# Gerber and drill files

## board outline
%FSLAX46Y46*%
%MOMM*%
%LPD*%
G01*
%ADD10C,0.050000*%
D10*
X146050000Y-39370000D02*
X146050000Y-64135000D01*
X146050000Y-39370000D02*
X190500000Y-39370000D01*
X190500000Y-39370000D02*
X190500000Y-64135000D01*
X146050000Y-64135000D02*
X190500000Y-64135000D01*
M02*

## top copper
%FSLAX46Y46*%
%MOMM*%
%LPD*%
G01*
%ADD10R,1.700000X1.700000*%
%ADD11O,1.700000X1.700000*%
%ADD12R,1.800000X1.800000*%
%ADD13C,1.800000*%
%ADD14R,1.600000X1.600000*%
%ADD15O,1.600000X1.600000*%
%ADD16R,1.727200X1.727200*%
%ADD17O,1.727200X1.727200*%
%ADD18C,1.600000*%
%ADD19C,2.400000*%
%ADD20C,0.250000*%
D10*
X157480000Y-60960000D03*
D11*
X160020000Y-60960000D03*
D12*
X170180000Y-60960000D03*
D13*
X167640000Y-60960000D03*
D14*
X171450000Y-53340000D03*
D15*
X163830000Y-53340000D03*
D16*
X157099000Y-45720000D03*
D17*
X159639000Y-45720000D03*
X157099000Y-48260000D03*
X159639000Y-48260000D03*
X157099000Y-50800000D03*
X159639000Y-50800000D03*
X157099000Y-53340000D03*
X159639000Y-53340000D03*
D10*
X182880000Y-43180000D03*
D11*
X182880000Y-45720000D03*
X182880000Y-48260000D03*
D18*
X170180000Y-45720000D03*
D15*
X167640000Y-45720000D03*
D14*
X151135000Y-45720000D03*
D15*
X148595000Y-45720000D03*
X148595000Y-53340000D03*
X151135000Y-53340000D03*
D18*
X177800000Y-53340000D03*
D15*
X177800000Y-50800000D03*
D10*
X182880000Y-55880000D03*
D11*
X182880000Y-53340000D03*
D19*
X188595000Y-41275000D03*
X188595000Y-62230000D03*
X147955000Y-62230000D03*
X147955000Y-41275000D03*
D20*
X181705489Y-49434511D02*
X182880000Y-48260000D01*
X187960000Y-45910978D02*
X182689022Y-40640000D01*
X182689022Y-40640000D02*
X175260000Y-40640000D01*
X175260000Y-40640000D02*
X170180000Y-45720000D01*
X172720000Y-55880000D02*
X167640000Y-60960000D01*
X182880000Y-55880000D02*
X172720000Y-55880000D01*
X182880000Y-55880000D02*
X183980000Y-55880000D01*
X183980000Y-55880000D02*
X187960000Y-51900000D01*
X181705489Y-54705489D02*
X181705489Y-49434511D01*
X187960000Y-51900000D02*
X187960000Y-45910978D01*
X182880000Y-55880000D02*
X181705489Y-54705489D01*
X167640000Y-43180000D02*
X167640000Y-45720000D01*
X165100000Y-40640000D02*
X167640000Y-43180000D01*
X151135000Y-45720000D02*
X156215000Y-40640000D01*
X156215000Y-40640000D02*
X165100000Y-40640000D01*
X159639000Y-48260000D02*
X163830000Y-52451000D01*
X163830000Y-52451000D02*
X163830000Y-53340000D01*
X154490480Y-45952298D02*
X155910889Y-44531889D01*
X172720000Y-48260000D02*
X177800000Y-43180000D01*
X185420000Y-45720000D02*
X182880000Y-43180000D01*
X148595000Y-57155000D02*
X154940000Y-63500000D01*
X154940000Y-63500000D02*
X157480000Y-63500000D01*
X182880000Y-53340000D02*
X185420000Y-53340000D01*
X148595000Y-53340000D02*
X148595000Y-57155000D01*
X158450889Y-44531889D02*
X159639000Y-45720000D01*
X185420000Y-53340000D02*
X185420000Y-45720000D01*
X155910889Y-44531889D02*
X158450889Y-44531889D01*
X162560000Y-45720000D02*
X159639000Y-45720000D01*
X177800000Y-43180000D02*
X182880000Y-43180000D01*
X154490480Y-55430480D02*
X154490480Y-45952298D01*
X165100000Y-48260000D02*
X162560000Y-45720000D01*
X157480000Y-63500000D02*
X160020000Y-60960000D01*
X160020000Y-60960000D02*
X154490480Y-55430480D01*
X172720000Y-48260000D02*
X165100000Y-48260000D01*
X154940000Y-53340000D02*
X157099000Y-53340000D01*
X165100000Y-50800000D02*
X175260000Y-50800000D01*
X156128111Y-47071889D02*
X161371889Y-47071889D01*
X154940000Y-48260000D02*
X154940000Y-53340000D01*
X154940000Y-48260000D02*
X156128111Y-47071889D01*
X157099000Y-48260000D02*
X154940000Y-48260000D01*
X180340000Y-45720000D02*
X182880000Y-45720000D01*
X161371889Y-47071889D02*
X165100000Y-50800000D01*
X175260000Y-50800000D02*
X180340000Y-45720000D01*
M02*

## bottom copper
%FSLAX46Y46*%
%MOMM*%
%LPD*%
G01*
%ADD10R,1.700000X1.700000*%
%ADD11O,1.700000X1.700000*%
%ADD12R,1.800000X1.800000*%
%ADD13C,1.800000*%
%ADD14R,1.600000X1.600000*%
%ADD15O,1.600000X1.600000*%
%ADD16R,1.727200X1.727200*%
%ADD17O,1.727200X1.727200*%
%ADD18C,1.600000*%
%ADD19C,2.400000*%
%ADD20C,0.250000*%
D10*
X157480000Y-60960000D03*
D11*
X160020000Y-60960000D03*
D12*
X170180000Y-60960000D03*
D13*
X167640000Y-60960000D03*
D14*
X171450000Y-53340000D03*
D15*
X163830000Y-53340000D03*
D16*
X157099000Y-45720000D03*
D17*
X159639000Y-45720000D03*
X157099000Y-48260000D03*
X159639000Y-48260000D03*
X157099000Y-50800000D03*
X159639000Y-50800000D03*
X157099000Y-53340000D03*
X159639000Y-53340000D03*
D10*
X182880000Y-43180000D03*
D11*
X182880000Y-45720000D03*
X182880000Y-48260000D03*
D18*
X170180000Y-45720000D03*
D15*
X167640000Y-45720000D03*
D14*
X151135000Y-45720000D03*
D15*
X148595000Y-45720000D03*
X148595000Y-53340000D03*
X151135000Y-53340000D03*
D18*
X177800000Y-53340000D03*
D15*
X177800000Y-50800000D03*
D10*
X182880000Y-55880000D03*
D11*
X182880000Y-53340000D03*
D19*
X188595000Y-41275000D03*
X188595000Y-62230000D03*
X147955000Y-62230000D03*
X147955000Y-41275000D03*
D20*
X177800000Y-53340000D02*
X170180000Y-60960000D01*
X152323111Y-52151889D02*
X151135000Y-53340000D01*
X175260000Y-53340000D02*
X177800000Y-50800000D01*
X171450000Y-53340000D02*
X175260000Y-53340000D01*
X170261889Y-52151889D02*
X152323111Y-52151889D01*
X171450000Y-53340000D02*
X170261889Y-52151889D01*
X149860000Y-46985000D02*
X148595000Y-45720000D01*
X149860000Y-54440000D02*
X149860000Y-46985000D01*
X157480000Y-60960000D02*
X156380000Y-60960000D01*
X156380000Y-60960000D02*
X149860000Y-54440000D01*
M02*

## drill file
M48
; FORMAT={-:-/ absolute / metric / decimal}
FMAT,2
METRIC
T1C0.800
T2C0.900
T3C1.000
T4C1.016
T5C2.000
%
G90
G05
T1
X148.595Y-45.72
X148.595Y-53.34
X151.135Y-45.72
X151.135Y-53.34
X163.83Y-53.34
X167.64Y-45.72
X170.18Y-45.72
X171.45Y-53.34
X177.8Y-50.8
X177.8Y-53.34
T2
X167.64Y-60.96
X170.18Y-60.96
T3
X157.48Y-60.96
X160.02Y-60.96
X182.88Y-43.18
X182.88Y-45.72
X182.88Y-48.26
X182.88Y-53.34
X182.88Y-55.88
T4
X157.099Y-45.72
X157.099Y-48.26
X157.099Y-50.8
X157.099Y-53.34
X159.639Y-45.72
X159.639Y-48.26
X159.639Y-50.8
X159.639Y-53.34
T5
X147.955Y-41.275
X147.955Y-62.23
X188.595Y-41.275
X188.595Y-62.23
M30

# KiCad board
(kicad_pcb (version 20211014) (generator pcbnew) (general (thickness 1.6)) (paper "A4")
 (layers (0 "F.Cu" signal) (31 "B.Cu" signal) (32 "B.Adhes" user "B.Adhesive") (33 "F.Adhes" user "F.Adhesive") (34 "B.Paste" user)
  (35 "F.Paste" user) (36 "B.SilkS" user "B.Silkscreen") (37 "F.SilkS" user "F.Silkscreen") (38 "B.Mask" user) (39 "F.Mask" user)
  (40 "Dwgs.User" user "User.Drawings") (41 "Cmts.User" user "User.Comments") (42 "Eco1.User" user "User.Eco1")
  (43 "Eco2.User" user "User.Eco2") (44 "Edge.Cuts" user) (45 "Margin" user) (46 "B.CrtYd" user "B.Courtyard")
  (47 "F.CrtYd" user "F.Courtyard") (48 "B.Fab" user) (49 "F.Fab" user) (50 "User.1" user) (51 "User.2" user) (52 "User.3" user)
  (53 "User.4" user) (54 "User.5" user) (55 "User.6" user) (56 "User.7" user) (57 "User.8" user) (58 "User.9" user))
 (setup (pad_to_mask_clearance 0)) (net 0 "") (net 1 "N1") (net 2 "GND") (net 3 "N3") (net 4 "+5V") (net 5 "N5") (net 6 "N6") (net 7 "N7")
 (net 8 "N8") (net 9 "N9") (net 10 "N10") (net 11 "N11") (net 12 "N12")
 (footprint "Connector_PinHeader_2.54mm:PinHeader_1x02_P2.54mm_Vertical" (layer "F.Cu") (at 157.48 60.96 90)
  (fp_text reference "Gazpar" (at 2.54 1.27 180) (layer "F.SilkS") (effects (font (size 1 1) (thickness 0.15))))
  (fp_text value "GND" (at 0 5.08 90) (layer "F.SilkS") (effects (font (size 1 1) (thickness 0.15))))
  (pad "1" thru_hole rect (at 0 0 90) (size 1.7 1.7) (drill 1) (layers *.Cu *.Mask) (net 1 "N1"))
  (pad "2" thru_hole oval (at 0 2.54 90) (size 1.7 1.7) (drill 1) (layers *.Cu *.Mask) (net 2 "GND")))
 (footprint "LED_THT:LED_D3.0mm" (layer "F.Cu") (at 170.18 60.96 180)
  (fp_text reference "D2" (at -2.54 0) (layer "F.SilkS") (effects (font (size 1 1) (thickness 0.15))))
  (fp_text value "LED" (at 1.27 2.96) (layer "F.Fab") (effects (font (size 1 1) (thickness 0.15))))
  (pad "1" thru_hole rect (at 0 0 180) (size 1.8 1.8) (drill 0.9) (layers *.Cu *.Mask) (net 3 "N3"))
  (pad "2" thru_hole circle (at 2.54 0 180) (size 1.8 1.8) (drill 0.9) (layers *.Cu *.Mask) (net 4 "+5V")))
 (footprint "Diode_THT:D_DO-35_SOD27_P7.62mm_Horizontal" (layer "F.Cu") (at 171.45 53.34 180)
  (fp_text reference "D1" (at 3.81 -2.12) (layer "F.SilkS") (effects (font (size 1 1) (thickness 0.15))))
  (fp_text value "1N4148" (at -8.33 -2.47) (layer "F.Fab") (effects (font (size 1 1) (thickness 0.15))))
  (pad "1" thru_hole rect (at 0 0 180) (size 1.6 1.6) (drill 0.8) (layers *.Cu *.Mask) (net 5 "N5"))
  (pad "2" thru_hole oval (at 7.62 0 180) (size 1.6 1.6) (drill 0.8) (layers *.Cu *.Mask) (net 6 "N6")))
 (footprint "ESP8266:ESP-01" (layer "F.Cu") (at 157.099 45.72)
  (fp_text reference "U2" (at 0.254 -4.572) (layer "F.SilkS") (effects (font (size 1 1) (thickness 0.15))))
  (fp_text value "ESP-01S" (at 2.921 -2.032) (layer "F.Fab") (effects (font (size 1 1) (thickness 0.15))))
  (pad "1" thru_hole rect locked (at 0 0) (size 1.7272 1.7272) (drill 1.016) (layers *.Cu *.Mask "F.SilkS") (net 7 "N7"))
  (pad "2" thru_hole oval locked (at 2.54 0) (size 1.7272 1.7272) (drill 1.016) (layers *.Cu *.Mask "F.SilkS") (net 2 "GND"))
  (pad "3" thru_hole oval locked (at 0 2.54) (size 1.7272 1.7272) (drill 1.016) (layers *.Cu *.Mask "F.SilkS") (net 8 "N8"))
  (pad "4" thru_hole oval locked (at 2.54 2.54) (size 1.7272 1.7272) (drill 1.016) (layers *.Cu *.Mask "F.SilkS") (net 6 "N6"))
  (pad "5" thru_hole oval locked (at 0 5.08) (size 1.7272 1.7272) (drill 1.016) (layers *.Cu *.Mask "F.SilkS") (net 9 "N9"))
  (pad "6" thru_hole oval locked (at 2.54 5.08) (size 1.7272 1.7272) (drill 1.016) (layers *.Cu *.Mask "F.SilkS") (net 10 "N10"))
  (pad "7" thru_hole oval locked (at 0 7.62) (size 1.7272 1.7272) (drill 1.016) (layers *.Cu *.Mask "F.SilkS") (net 8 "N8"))
  (pad "8" thru_hole oval locked (at 2.54 7.62) (size 1.7272 1.7272) (drill 1.016) (layers *.Cu *.Mask "F.SilkS") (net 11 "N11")))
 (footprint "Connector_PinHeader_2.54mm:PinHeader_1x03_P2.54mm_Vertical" (layer "F.Cu") (at 182.88 43.18)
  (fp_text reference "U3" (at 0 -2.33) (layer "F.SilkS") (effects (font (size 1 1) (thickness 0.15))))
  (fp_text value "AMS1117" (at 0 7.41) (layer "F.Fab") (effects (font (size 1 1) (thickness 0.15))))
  (pad "1" thru_hole rect (at 0 0) (size 1.7 1.7) (drill 1) (layers *.Cu *.Mask) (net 2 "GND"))
  (pad "2" thru_hole oval (at 0 2.54) (size 1.7 1.7) (drill 1) (layers *.Cu *.Mask) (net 8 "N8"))
  (pad "3" thru_hole oval (at 0 5.08) (size 1.7 1.7) (drill 1) (layers *.Cu *.Mask) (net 4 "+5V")))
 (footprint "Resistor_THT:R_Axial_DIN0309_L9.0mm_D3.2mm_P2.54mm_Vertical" (layer "F.Cu") (at 170.18 45.72 180)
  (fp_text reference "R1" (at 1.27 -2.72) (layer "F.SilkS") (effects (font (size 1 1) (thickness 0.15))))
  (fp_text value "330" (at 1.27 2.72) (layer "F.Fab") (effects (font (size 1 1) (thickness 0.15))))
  (pad "1" thru_hole circle (at 0 0 180) (size 1.6 1.6) (drill 0.8) (layers *.Cu *.Mask) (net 4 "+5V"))
  (pad "2" thru_hole oval (at 2.54 0 180) (size 1.6 1.6) (drill 0.8) (layers *.Cu *.Mask) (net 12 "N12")))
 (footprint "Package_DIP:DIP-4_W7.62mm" (layer "F.Cu") (at 151.135 45.72 -90)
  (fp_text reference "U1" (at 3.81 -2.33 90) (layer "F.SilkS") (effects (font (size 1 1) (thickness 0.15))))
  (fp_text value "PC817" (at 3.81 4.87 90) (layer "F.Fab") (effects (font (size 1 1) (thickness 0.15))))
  (pad "1" thru_hole rect (at 0 0 270) (size 1.6 1.6) (drill 0.8) (layers *.Cu *.Mask) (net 12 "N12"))
  (pad "2" thru_hole oval (at 0 2.54 270) (size 1.6 1.6) (drill 0.8) (layers *.Cu *.Mask) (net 1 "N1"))
  (pad "3" thru_hole oval (at 7.62 2.54 270) (size 1.6 1.6) (drill 0.8) (layers *.Cu *.Mask) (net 2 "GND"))
  (pad "4" thru_hole oval (at 7.62 0 270) (size 1.6 1.6) (drill 0.8) (layers *.Cu *.Mask) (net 5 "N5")))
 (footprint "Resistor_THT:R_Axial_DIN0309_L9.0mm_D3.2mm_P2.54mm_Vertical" (layer "F.Cu") (at 177.8 53.34 90)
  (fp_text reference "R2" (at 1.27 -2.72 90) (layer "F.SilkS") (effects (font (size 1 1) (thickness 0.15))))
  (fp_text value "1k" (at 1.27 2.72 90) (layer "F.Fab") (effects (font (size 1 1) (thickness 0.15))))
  (pad "1" thru_hole circle (at 0 0 90) (size 1.6 1.6) (drill 0.8) (layers *.Cu *.Mask) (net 3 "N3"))
  (pad "2" thru_hole oval (at 2.54 0 90) (size 1.6 1.6) (drill 0.8) (layers *.Cu *.Mask) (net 5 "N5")))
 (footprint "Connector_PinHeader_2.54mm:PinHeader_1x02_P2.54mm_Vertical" (layer "F.Cu") (at 182.88 55.88 180)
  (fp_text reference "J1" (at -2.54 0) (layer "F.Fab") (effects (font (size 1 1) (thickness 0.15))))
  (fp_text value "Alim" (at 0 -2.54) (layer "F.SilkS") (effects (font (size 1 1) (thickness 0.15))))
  (pad "1" thru_hole rect (at 0 0 180) (size 1.7 1.7) (drill 1) (layers *.Cu *.Mask) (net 4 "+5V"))
  (pad "2" thru_hole oval (at 0 2.54 180) (size 1.7 1.7) (drill 1) (layers *.Cu *.Mask) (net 2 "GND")))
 (gr_line (start 146.05 39.37) (end 146.05 64.135) (layer "Edge.Cuts") (width 0.05))
 (gr_line (start 146.05 39.37) (end 190.5 39.37) (layer "Edge.Cuts") (width 0.05))
 (gr_line (start 190.5 39.37) (end 190.5 64.135) (layer "Edge.Cuts") (width 0.05))
 (gr_line (start 146.05 64.135) (end 190.5 64.135) (layer "Edge.Cuts") (width 0.05))
 (via (at 188.595 41.275) (size 2.4) (drill 2) (layers "F.Cu" "B.Cu") (free) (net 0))
 (via (at 188.595 62.23) (size 2.4) (drill 2) (layers "F.Cu" "B.Cu") (free) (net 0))
 (via (at 147.955 62.23) (size 2.4) (drill 2) (layers "F.Cu" "B.Cu") (free) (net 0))
 (via (at 147.955 41.275) (size 2.4) (drill 2) (layers "F.Cu" "B.Cu") (free) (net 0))
 (segment (start 181.705489 49.434511) (end 182.88 48.26) (width 0.25) (layer "F.Cu") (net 4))
 (segment (start 187.96 45.910978) (end 182.689022 40.64) (width 0.25) (layer "F.Cu") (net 4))
 (segment (start 182.689022 40.64) (end 175.26 40.64) (width 0.25) (layer "F.Cu") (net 4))
 (segment (start 175.26 40.64) (end 170.18 45.72) (width 0.25) (layer "F.Cu") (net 4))
 (segment (start 172.72 55.88) (end 167.64 60.96) (width 0.25) (layer "F.Cu") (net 4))
 (segment (start 182.88 55.88) (end 172.72 55.88) (width 0.25) (layer "F.Cu") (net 4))
 (segment (start 182.88 55.88) (end 183.98 55.88) (width 0.25) (layer "F.Cu") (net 4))
 (segment (start 183.98 55.88) (end 187.96 51.9) (width 0.25) (layer "F.Cu") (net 4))
 (segment (start 181.705489 54.705489) (end 181.705489 49.434511) (width 0.25) (layer "F.Cu") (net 4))
 (segment (start 187.96 51.9) (end 187.96 45.910978) (width 0.25) (layer "F.Cu") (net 4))
 (segment (start 182.88 55.88) (end 181.705489 54.705489) (width 0.25) (layer "F.Cu") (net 4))
 (segment (start 167.64 43.18) (end 167.64 45.72) (width 0.25) (layer "F.Cu") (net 12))
 (segment (start 165.1 40.64) (end 167.64 43.18) (width 0.25) (layer "F.Cu") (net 12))
 (segment (start 151.135 45.72) (end 156.215 40.64) (width 0.25) (layer "F.Cu") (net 12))
 (segment (start 156.215 40.64) (end 165.1 40.64) (width 0.25) (layer "F.Cu") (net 12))
 (segment (start 177.8 53.34) (end 170.18 60.96) (width 0.25) (layer "B.Cu") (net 3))
 (segment (start 152.323111 52.151889) (end 151.135 53.34) (width 0.25) (layer "B.Cu") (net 5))
 (segment (start 175.26 53.34) (end 177.8 50.8) (width 0.25) (layer "B.Cu") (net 5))
 (segment (start 171.45 53.34) (end 175.26 53.34) (width 0.25) (layer "B.Cu") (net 5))
 (segment (start 170.261889 52.151889) (end 152.323111 52.151889) (width 0.25) (layer "B.Cu") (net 5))
 (segment (start 171.45 53.34) (end 170.261889 52.151889) (width 0.25) (layer "B.Cu") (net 5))
 (segment (start 149.86 46.985) (end 148.595 45.72) (width 0.25) (layer "B.Cu") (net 1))
 (segment (start 149.86 54.44) (end 149.86 46.985) (width 0.25) (layer "B.Cu") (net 1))
 (segment (start 157.48 60.96) (end 156.38 60.96) (width 0.25) (layer "B.Cu") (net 1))
 (segment (start 156.38 60.96) (end 149.86 54.44) (width 0.25) (layer "B.Cu") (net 1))
 (segment (start 159.639 48.26) (end 163.83 52.451) (width 0.25) (layer "F.Cu") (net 6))
 (segment (start 163.83 52.451) (end 163.83 53.34) (width 0.25) (layer "F.Cu") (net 6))
 (segment (start 154.49048 45.952298) (end 155.910889 44.531889) (width 0.25) (layer "F.Cu") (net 2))
 (segment (start 172.72 48.26) (end 177.8 43.18) (width 0.25) (layer "F.Cu") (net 2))
 (segment (start 185.42 45.72) (end 182.88 43.18) (width 0.25) (layer "F.Cu") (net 2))
 (segment (start 148.595 57.155) (end 154.94 63.5) (width 0.25) (layer "F.Cu") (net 2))
 (segment (start 154.94 63.5) (end 157.48 63.5) (width 0.25) (layer "F.Cu") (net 2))
 (segment (start 182.88 53.34) (end 185.42 53.34) (width 0.25) (layer "F.Cu") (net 2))
 (segment (start 148.595 53.34) (end 148.595 57.155) (width 0.25) (layer "F.Cu") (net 2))
 (segment (start 158.450889 44.531889) (end 159.639 45.72) (width 0.25) (layer "F.Cu") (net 2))
 (segment (start 185.42 53.34) (end 185.42 45.72) (width 0.25) (layer "F.Cu") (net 2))
 (segment (start 155.910889 44.531889) (end 158.450889 44.531889) (width 0.25) (layer "F.Cu") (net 2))
 (segment (start 162.56 45.72) (end 159.639 45.72) (width 0.25) (layer "F.Cu") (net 2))
 (segment (start 177.8 43.18) (end 182.88 43.18) (width 0.25) (layer "F.Cu") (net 2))
 (segment (start 154.49048 55.43048) (end 154.49048 45.952298) (width 0.25) (layer "F.Cu") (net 2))
 (segment (start 165.1 48.26) (end 162.56 45.72) (width 0.25) (layer "F.Cu") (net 2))
 (segment (start 157.48 63.5) (end 160.02 60.96) (width 0.25) (layer "F.Cu") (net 2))
 (segment (start 160.02 60.96) (end 154.49048 55.43048) (width 0.25) (layer "F.Cu") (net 2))
 (segment (start 172.72 48.26) (end 165.1 48.26) (width 0.25) (layer "F.Cu") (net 2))
 (segment (start 154.94 53.34) (end 157.099 53.34) (width 0.25) (layer "F.Cu") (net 8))
 (segment (start 165.1 50.8) (end 175.26 50.8) (width 0.25) (layer "F.Cu") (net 8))
 (segment (start 156.128111 47.071889) (end 161.371889 47.071889) (width 0.25) (layer "F.Cu") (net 8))
 (segment (start 154.94 48.26) (end 154.94 53.34) (width 0.25) (layer "F.Cu") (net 8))
 (segment (start 154.94 48.26) (end 156.128111 47.071889) (width 0.25) (layer "F.Cu") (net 8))
 (segment (start 157.099 48.26) (end 154.94 48.26) (width 0.25) (layer "F.Cu") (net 8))
 (segment (start 180.34 45.72) (end 182.88 45.72) (width 0.25) (layer "F.Cu") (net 8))
 (segment (start 161.371889 47.071889) (end 165.1 50.8) (width 0.25) (layer "F.Cu") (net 8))
 (segment (start 175.26 50.8) (end 180.34 45.72) (width 0.25) (layer "F.Cu") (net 8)))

